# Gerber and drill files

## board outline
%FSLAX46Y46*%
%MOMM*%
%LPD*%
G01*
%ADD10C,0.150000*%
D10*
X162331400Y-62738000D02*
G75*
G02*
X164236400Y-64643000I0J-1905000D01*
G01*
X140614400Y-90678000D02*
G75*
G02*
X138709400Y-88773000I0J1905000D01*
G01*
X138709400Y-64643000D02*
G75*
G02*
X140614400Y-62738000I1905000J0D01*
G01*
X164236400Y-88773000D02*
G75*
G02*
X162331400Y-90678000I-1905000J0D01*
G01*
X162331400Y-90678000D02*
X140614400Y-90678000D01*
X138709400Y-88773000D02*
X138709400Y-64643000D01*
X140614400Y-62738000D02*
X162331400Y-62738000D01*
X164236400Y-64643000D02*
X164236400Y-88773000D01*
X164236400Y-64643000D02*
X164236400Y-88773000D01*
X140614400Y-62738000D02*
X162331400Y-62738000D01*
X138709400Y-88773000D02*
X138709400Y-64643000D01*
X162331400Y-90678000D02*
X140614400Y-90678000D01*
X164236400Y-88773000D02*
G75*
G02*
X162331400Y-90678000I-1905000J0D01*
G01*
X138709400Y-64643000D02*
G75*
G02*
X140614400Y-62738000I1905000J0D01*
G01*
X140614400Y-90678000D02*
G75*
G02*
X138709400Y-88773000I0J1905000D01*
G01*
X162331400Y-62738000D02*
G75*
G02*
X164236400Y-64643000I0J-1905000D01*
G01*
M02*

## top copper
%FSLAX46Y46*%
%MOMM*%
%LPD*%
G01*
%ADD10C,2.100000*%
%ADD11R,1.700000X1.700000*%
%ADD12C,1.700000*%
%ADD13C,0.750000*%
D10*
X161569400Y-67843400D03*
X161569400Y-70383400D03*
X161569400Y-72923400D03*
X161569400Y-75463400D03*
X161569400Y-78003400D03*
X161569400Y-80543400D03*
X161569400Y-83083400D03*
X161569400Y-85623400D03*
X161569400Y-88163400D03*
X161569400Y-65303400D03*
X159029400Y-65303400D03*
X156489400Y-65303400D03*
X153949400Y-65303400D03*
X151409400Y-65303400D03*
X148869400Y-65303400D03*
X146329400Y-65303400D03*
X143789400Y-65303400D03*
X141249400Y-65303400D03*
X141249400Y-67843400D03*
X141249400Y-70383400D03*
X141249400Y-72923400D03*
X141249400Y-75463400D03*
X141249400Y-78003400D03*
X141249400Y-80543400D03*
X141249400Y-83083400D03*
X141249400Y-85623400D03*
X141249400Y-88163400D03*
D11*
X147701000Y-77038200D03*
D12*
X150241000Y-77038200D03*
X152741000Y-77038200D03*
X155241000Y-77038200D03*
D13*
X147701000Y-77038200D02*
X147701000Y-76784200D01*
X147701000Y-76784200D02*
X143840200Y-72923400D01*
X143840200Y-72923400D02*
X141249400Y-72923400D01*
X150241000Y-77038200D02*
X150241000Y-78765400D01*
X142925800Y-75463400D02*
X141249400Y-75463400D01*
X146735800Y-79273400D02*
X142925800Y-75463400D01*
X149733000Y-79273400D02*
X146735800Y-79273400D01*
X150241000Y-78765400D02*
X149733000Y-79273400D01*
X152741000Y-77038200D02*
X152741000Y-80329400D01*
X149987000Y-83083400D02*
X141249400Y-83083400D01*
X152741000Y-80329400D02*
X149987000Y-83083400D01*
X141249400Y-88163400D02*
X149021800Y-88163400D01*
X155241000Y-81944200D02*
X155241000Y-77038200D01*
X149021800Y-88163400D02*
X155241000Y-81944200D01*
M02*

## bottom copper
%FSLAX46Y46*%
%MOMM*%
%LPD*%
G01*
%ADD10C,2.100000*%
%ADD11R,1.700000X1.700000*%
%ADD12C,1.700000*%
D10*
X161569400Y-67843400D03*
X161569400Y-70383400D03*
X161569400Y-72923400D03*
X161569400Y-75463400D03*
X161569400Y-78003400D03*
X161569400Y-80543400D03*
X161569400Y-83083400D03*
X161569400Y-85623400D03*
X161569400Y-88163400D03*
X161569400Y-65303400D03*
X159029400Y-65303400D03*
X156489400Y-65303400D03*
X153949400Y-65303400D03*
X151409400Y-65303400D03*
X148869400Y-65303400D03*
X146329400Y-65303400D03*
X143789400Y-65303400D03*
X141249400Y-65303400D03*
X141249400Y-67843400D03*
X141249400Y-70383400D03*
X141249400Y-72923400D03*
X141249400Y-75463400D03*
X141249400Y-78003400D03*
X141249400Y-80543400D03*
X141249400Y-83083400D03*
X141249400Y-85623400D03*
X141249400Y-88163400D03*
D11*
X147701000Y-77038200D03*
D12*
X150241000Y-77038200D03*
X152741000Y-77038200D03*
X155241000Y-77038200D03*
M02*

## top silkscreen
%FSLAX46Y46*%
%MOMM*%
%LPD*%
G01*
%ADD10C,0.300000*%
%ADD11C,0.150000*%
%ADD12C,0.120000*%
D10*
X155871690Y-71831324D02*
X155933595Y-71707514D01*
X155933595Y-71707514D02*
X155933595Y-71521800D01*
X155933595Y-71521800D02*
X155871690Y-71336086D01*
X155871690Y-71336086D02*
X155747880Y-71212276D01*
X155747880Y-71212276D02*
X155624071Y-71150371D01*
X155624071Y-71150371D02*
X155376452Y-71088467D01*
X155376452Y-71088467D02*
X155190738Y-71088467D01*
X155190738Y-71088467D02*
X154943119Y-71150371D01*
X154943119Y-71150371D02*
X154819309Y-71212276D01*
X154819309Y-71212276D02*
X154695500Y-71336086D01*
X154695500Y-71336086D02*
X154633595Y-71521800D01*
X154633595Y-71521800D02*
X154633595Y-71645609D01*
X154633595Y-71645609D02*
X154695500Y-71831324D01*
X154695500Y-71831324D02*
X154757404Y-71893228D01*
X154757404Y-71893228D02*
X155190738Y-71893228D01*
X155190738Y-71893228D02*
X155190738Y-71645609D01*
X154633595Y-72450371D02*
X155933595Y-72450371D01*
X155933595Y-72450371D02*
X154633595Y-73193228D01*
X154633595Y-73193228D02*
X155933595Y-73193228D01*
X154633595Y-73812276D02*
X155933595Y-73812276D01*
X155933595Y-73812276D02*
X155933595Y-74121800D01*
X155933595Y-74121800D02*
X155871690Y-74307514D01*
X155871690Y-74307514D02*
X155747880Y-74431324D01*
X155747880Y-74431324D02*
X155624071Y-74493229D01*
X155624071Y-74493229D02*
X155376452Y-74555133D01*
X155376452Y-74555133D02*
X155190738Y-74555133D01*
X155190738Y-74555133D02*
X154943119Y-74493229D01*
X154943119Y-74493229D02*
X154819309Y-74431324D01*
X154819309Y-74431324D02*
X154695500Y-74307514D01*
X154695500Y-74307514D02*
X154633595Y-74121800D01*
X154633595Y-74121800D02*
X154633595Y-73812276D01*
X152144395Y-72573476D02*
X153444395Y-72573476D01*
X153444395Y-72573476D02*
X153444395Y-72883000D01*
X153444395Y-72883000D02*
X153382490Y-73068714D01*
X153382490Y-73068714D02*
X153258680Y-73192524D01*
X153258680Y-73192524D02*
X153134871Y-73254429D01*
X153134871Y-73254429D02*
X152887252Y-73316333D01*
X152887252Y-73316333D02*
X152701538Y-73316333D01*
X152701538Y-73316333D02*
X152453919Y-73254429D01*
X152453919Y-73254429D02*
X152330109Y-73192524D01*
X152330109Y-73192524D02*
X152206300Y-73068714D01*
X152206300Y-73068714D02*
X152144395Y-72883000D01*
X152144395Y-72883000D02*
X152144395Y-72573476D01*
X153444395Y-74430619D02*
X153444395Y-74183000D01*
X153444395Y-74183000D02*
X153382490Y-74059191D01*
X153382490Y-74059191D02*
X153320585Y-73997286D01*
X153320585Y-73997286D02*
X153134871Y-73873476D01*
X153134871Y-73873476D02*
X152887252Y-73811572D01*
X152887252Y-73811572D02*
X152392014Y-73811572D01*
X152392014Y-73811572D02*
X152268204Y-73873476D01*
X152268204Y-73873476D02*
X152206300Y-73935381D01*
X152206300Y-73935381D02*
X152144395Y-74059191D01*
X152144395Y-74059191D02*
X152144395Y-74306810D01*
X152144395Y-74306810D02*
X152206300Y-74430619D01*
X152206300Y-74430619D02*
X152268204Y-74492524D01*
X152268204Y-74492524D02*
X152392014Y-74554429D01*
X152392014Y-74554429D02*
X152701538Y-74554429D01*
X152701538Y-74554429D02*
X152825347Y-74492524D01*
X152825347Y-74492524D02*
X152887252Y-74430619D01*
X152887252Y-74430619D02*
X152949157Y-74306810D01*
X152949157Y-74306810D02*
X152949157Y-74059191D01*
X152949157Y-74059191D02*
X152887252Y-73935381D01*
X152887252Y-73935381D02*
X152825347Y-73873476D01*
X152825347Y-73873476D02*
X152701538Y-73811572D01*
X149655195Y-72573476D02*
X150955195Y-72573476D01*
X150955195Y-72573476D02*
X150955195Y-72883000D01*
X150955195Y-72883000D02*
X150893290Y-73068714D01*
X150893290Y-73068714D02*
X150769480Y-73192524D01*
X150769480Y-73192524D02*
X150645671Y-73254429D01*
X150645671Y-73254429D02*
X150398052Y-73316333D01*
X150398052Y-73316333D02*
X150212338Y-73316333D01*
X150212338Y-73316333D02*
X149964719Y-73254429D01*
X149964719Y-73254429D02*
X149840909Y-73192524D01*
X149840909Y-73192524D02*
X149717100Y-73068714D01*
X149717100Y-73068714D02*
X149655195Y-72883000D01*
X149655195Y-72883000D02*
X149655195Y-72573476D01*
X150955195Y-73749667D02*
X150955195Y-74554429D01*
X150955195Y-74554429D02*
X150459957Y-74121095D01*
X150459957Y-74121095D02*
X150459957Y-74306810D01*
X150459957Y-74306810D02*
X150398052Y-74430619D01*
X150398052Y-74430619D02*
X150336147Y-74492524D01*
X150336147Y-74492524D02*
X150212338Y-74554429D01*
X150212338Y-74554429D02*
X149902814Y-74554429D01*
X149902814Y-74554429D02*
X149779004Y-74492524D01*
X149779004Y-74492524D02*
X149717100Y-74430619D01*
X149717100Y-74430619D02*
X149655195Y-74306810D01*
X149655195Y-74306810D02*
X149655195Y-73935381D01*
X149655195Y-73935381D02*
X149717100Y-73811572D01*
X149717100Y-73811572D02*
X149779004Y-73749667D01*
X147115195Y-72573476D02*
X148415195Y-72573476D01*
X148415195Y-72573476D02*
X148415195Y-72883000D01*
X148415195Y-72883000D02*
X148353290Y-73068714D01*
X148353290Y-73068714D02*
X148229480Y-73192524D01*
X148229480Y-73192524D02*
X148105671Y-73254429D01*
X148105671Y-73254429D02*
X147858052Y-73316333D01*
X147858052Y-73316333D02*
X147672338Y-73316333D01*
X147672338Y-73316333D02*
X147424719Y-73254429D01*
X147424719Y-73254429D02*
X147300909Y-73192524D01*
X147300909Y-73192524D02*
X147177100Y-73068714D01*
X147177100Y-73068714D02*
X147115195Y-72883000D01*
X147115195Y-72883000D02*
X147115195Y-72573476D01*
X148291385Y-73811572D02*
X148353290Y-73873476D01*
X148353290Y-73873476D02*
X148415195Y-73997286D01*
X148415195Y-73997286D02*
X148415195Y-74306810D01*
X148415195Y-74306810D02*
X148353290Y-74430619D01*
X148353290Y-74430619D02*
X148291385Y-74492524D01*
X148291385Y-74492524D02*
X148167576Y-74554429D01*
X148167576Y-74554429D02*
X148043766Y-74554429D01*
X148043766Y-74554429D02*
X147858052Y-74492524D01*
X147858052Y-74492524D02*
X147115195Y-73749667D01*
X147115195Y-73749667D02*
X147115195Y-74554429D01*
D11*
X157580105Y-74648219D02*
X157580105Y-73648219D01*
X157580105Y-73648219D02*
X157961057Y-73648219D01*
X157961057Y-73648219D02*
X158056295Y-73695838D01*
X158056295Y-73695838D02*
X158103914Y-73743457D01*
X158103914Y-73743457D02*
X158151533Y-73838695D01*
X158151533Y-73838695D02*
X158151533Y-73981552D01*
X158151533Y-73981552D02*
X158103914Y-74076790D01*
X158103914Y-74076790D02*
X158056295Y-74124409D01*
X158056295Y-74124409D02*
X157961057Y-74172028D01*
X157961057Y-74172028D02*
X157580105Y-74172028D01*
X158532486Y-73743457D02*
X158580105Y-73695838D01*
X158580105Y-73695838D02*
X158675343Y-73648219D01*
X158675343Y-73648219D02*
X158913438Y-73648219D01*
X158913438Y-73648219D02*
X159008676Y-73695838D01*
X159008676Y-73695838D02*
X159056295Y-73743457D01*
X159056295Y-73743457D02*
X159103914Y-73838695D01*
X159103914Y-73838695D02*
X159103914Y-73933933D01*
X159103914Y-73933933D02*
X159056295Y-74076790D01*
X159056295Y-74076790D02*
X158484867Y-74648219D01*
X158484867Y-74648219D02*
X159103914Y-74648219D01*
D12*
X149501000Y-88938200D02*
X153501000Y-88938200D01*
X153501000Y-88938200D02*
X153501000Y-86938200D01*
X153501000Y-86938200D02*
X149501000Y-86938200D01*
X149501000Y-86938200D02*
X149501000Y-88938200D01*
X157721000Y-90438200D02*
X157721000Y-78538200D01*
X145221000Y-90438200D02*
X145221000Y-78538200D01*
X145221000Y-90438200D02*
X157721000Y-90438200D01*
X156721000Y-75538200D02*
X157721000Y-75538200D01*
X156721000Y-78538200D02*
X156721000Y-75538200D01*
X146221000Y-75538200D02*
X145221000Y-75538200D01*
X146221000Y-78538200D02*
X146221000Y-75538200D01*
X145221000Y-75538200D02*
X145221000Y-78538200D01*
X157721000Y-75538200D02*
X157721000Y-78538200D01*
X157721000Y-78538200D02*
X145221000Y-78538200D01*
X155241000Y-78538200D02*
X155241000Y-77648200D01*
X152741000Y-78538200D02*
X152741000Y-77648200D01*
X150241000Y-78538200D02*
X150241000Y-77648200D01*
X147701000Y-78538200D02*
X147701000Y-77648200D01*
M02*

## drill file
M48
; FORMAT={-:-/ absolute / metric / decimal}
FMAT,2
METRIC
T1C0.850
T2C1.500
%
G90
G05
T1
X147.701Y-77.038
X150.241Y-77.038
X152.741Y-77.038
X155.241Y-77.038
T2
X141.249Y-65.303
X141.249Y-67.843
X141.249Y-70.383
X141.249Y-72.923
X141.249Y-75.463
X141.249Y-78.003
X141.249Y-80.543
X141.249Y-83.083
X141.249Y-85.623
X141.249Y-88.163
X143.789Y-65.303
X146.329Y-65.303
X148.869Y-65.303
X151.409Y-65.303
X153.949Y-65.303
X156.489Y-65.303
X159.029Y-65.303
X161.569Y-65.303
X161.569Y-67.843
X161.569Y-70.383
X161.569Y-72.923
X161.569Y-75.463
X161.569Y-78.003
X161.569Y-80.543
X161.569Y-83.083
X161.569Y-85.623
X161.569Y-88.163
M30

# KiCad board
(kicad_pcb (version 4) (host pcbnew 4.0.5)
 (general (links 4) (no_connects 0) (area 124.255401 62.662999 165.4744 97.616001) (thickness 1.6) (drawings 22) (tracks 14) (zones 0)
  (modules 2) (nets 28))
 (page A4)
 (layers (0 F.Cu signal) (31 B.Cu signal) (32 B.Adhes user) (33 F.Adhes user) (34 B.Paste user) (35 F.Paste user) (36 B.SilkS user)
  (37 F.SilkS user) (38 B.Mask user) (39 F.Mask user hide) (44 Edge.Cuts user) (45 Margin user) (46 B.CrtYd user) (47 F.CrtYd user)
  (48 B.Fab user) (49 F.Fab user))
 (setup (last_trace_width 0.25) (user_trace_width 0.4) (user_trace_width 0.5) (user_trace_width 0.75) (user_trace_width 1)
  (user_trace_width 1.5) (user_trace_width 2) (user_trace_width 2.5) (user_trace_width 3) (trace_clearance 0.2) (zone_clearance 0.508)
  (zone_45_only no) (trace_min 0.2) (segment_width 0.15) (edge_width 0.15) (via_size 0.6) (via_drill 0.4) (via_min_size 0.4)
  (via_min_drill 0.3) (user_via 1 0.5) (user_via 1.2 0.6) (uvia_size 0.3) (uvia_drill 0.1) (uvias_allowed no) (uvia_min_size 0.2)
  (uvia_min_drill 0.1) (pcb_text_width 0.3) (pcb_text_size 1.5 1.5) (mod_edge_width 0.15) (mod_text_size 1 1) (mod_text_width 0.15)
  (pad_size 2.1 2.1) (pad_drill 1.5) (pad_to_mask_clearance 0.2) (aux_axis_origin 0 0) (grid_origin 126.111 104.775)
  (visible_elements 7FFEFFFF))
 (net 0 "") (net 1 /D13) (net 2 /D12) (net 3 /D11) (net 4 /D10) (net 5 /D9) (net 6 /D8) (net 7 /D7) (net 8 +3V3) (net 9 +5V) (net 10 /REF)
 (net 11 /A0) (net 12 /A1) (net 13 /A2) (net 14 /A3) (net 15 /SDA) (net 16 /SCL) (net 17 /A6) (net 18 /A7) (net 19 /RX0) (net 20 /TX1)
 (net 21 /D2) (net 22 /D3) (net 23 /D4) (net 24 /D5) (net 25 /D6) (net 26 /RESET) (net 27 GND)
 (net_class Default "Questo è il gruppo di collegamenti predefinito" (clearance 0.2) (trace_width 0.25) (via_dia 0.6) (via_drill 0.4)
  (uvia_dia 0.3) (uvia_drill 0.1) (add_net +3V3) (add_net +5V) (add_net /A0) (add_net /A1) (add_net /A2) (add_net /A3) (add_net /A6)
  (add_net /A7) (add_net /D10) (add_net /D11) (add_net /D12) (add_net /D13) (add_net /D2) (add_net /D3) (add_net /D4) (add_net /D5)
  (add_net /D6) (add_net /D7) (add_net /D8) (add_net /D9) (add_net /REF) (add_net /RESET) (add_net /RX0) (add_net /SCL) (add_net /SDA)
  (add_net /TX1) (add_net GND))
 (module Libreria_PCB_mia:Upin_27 (layer B.Cu) (at 161.5694 88.1634 180)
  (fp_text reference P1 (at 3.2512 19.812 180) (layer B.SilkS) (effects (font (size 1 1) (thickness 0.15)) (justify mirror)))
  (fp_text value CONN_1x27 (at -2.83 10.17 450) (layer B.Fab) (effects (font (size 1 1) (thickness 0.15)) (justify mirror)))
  (pad 9 thru_hole circle (at 0 20.32 180) (size 2.1 2.1) (drill 1.5) (layers *.Cu *.Mask) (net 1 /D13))
  (pad 8 thru_hole circle (at 0 17.78 180) (size 2.1 2.1) (drill 1.5) (layers *.Cu *.Mask) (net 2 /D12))
  (pad 7 thru_hole circle (at 0 15.24 180) (size 2.1 2.1) (drill 1.5) (layers *.Cu *.Mask) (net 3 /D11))
  (pad 6 thru_hole circle (at 0 12.7 180) (size 2.1 2.1) (drill 1.5) (layers *.Cu *.Mask) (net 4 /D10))
  (pad 5 thru_hole circle (at 0 10.16 180) (size 2.1 2.1) (drill 1.5) (layers *.Cu *.Mask) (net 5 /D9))
  (pad 4 thru_hole circle (at 0 7.62 180) (size 2.1 2.1) (drill 1.5) (layers *.Cu *.Mask) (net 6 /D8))
  (pad 3 thru_hole circle (at 0 5.08 180) (size 2.1 2.1) (drill 1.5) (layers *.Cu *.Mask) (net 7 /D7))
  (pad 2 thru_hole circle (at 0 2.54 180) (size 2.1 2.1) (drill 1.5) (layers *.Cu *.Mask) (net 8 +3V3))
  (pad 1 thru_hole circle (at 0 0 180) (size 2.1 2.1) (drill 1.5) (layers *.Cu *.Mask) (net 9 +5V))
  (pad 10 thru_hole circle (at 0 22.86 180) (size 2.1 2.1) (drill 1.5) (layers *.Cu *.Mask) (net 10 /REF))
  (pad 11 thru_hole circle (at 2.54 22.86 180) (size 2.1 2.1) (drill 1.5) (layers *.Cu *.Mask) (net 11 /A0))
  (pad 12 thru_hole circle (at 5.08 22.86 180) (size 2.1 2.1) (drill 1.5) (layers *.Cu *.Mask) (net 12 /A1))
  (pad 13 thru_hole circle (at 7.62 22.86 180) (size 2.1 2.1) (drill 1.5) (layers *.Cu *.Mask) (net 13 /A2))
  (pad 14 thru_hole circle (at 10.16 22.86 180) (size 2.1 2.1) (drill 1.5) (layers *.Cu *.Mask) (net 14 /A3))
  (pad 15 thru_hole circle (at 12.7 22.86 180) (size 2.1 2.1) (drill 1.5) (layers *.Cu *.Mask) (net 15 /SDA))
  (pad 16 thru_hole circle (at 15.24 22.86 180) (size 2.1 2.1) (drill 1.5) (layers *.Cu *.Mask) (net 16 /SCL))
  (pad 17 thru_hole circle (at 17.78 22.86 180) (size 2.1 2.1) (drill 1.5) (layers *.Cu *.Mask) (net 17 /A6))
  (pad 18 thru_hole circle (at 20.32 22.86 180) (size 2.1 2.1) (drill 1.5) (layers *.Cu *.Mask) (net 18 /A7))
  (pad 19 thru_hole circle (at 20.32 20.32 180) (size 2.1 2.1) (drill 1.5) (layers *.Cu *.Mask) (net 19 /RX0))
  (pad 20 thru_hole circle (at 20.32 17.78 180) (size 2.1 2.1) (drill 1.5) (layers *.Cu *.Mask) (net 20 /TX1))
  (pad 21 thru_hole circle (at 20.32 15.24 180) (size 2.1 2.1) (drill 1.5) (layers *.Cu *.Mask) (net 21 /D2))
  (pad 22 thru_hole circle (at 20.32 12.7 180) (size 2.1 2.1) (drill 1.5) (layers *.Cu *.Mask) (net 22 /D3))
  (pad 23 thru_hole circle (at 20.32 10.16 180) (size 2.1 2.1) (drill 1.5) (layers *.Cu *.Mask) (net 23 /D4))
  (pad 24 thru_hole circle (at 20.32 7.62 180) (size 2.1 2.1) (drill 1.5) (layers *.Cu *.Mask) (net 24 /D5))
  (pad 25 thru_hole circle (at 20.32 5.08 180) (size 2.1 2.1) (drill 1.5) (layers *.Cu *.Mask) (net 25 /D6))
  (pad 26 thru_hole circle (at 20.32 2.54 180) (size 2.1 2.1) (drill 1.5) (layers *.Cu *.Mask) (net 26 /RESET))
  (pad 27 thru_hole circle (at 20.32 0 180) (size 2.1 2.1) (drill 1.5) (layers *.Cu *.Mask) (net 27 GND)))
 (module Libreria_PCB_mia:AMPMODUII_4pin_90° (layer F.Cu) (at 147.701 77.0382)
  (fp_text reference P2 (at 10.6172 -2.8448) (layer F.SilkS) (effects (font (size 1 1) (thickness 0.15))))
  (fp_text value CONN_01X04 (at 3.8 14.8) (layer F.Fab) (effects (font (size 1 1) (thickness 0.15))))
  (fp_line (start 1.8 11.9) (end 5.8 11.9) (layer F.SilkS) (width 0.12))
  (fp_line (start 5.8 11.9) (end 5.8 9.9) (layer F.SilkS) (width 0.12))
  (fp_line (start 5.8 9.9) (end 1.8 9.9) (layer F.SilkS) (width 0.12))
  (fp_line (start 1.8 9.9) (end 1.8 11.9) (layer F.SilkS) (width 0.12))
  (fp_line (start 10.02 13.4) (end 10.02 1.5) (layer F.SilkS) (width 0.12))
  (fp_line (start -2.48 13.4) (end -2.48 1.5) (layer F.SilkS) (width 0.12))
  (fp_line (start -2.48 13.4) (end 10.02 13.4) (layer F.SilkS) (width 0.12))
  (fp_line (start 9.02 -1.5) (end 10.02 -1.5) (layer F.SilkS) (width 0.12))
  (fp_line (start 9.02 1.5) (end 9.02 -1.5) (layer F.SilkS) (width 0.12))
  (fp_line (start -1.48 -1.5) (end -2.48 -1.5) (layer F.SilkS) (width 0.12))
  (fp_line (start -1.48 1.5) (end -1.48 -1.5) (layer F.SilkS) (width 0.12))
  (fp_line (start -2.48 -1.5) (end -2.48 1.5) (layer F.SilkS) (width 0.12))
  (fp_line (start 10.02 -1.5) (end 10.02 1.5) (layer F.SilkS) (width 0.12))
  (fp_line (start 10.02 1.5) (end -2.48 1.5) (layer F.SilkS) (width 0.12))
  (fp_line (start 7.54 1.5) (end 7.54 0.61) (layer F.SilkS) (width 0.12))
  (fp_line (start 5.04 1.5) (end 5.04 0.61) (layer F.SilkS) (width 0.12))
  (fp_line (start 2.54 1.5) (end 2.54 0.61) (layer F.SilkS) (width 0.12))
  (fp_line (start 0 1.5) (end 0 0.61) (layer F.SilkS) (width 0.12))
  (pad 1 thru_hole rect (at 0 0) (size 1.7 1.7) (drill 0.85) (layers *.Cu *.Mask) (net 21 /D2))
  (pad 2 thru_hole circle (at 2.54 0) (size 1.7 1.7) (drill 0.85) (layers *.Cu *.Mask) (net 22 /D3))
  (pad 3 thru_hole circle (at 5.04 0) (size 1.7 1.7) (drill 0.85) (layers *.Cu *.Mask) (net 25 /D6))
  (pad 4 thru_hole circle (at 7.54 0) (size 1.7 1.7) (drill 0.85) (layers *.Cu *.Mask) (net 27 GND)))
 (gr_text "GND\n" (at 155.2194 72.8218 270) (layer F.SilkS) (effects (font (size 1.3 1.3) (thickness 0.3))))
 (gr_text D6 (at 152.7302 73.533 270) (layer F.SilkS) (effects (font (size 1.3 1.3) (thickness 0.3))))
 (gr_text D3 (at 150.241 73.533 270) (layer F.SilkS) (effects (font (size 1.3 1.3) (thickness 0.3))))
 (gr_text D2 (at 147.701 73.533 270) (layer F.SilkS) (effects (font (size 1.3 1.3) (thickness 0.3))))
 (gr_arc (start 162.3314 64.643) (end 162.3314 62.738) (angle 90) (layer Edge.Cuts) (width 0.15))
 (gr_arc (start 140.6144 88.773) (end 140.6144 90.678) (angle 90) (layer Edge.Cuts) (width 0.15))
 (gr_arc (start 140.6144 64.643) (end 138.7094 64.643) (angle 90) (layer Edge.Cuts) (width 0.15))
 (gr_arc (start 162.3314 88.773) (end 164.2364 88.773) (angle 90) (layer Edge.Cuts) (width 0.15))
 (gr_line (start 162.3314 90.678) (end 140.6144 90.678) (angle 90) (layer Edge.Cuts) (width 0.15))
 (gr_line (start 138.7094 88.773) (end 138.7094 64.643) (angle 90) (layer Edge.Cuts) (width 0.15))
 (gr_line (start 140.6144 62.738) (end 162.3314 62.738) (angle 90) (layer Edge.Cuts) (width 0.15))
 (gr_line (start 164.2364 64.643) (end 164.2364 88.773) (angle 90) (layer Edge.Cuts) (width 0.15))
 (gr_line (start 164.2364 64.643) (end 164.2364 88.773) (angle 90) (layer Edge.Cuts) (width 0.15))
 (gr_line (start 140.6144 62.738) (end 162.3314 62.738) (angle 90) (layer Edge.Cuts) (width 0.15))
 (gr_line (start 138.7094 88.773) (end 138.7094 64.643) (angle 90) (layer Edge.Cuts) (width 0.15))
 (gr_line (start 162.3314 90.678) (end 140.6144 90.678) (angle 90) (layer Edge.Cuts) (width 0.15))
 (gr_arc (start 162.3314 88.773) (end 164.2364 88.773) (angle 90) (layer Edge.Cuts) (width 0.15))
 (gr_arc (start 140.6144 64.643) (end 138.7094 64.643) (angle 90) (layer Edge.Cuts) (width 0.15))
 (gr_arc (start 140.6144 88.773) (end 140.6144 90.678) (angle 90) (layer Edge.Cuts) (width 0.15))
 (gr_arc (start 162.3314 64.643) (end 162.3314 62.738) (angle 90) (layer Edge.Cuts) (width 0.15))
 (segment (start 147.701 77.0382) (end 147.701 76.7842) (width 0.75) (layer F.Cu) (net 21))
 (segment (start 147.701 76.7842) (end 143.8402 72.9234) (width 0.75) (layer F.Cu) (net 21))
 (segment (start 143.8402 72.9234) (end 141.2494 72.9234) (width 0.75) (layer F.Cu) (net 21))
 (segment (start 150.241 77.0382) (end 150.241 78.7654) (width 0.75) (layer F.Cu) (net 22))
 (segment (start 142.9258 75.4634) (end 141.2494 75.4634) (width 0.75) (layer F.Cu) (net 22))
 (segment (start 146.7358 79.2734) (end 142.9258 75.4634) (width 0.75) (layer F.Cu) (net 22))
 (segment (start 149.733 79.2734) (end 146.7358 79.2734) (width 0.75) (layer F.Cu) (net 22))
 (segment (start 150.241 78.7654) (end 149.733 79.2734) (width 0.75) (layer F.Cu) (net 22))
 (segment (start 152.741 77.0382) (end 152.741 80.3294) (width 0.75) (layer F.Cu) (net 25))
 (segment (start 149.987 83.0834) (end 141.2494 83.0834) (width 0.75) (layer F.Cu) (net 25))
 (segment (start 152.741 80.3294) (end 149.987 83.0834) (width 0.75) (layer F.Cu) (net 25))
 (segment (start 141.2494 88.1634) (end 149.0218 88.1634) (width 0.75) (layer F.Cu) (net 27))
 (segment (start 155.241 81.9442) (end 155.241 77.0382) (width 0.75) (layer F.Cu) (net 27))
 (segment (start 149.0218 88.1634) (end 155.241 81.9442) (width 0.75) (layer F.Cu) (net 27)))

